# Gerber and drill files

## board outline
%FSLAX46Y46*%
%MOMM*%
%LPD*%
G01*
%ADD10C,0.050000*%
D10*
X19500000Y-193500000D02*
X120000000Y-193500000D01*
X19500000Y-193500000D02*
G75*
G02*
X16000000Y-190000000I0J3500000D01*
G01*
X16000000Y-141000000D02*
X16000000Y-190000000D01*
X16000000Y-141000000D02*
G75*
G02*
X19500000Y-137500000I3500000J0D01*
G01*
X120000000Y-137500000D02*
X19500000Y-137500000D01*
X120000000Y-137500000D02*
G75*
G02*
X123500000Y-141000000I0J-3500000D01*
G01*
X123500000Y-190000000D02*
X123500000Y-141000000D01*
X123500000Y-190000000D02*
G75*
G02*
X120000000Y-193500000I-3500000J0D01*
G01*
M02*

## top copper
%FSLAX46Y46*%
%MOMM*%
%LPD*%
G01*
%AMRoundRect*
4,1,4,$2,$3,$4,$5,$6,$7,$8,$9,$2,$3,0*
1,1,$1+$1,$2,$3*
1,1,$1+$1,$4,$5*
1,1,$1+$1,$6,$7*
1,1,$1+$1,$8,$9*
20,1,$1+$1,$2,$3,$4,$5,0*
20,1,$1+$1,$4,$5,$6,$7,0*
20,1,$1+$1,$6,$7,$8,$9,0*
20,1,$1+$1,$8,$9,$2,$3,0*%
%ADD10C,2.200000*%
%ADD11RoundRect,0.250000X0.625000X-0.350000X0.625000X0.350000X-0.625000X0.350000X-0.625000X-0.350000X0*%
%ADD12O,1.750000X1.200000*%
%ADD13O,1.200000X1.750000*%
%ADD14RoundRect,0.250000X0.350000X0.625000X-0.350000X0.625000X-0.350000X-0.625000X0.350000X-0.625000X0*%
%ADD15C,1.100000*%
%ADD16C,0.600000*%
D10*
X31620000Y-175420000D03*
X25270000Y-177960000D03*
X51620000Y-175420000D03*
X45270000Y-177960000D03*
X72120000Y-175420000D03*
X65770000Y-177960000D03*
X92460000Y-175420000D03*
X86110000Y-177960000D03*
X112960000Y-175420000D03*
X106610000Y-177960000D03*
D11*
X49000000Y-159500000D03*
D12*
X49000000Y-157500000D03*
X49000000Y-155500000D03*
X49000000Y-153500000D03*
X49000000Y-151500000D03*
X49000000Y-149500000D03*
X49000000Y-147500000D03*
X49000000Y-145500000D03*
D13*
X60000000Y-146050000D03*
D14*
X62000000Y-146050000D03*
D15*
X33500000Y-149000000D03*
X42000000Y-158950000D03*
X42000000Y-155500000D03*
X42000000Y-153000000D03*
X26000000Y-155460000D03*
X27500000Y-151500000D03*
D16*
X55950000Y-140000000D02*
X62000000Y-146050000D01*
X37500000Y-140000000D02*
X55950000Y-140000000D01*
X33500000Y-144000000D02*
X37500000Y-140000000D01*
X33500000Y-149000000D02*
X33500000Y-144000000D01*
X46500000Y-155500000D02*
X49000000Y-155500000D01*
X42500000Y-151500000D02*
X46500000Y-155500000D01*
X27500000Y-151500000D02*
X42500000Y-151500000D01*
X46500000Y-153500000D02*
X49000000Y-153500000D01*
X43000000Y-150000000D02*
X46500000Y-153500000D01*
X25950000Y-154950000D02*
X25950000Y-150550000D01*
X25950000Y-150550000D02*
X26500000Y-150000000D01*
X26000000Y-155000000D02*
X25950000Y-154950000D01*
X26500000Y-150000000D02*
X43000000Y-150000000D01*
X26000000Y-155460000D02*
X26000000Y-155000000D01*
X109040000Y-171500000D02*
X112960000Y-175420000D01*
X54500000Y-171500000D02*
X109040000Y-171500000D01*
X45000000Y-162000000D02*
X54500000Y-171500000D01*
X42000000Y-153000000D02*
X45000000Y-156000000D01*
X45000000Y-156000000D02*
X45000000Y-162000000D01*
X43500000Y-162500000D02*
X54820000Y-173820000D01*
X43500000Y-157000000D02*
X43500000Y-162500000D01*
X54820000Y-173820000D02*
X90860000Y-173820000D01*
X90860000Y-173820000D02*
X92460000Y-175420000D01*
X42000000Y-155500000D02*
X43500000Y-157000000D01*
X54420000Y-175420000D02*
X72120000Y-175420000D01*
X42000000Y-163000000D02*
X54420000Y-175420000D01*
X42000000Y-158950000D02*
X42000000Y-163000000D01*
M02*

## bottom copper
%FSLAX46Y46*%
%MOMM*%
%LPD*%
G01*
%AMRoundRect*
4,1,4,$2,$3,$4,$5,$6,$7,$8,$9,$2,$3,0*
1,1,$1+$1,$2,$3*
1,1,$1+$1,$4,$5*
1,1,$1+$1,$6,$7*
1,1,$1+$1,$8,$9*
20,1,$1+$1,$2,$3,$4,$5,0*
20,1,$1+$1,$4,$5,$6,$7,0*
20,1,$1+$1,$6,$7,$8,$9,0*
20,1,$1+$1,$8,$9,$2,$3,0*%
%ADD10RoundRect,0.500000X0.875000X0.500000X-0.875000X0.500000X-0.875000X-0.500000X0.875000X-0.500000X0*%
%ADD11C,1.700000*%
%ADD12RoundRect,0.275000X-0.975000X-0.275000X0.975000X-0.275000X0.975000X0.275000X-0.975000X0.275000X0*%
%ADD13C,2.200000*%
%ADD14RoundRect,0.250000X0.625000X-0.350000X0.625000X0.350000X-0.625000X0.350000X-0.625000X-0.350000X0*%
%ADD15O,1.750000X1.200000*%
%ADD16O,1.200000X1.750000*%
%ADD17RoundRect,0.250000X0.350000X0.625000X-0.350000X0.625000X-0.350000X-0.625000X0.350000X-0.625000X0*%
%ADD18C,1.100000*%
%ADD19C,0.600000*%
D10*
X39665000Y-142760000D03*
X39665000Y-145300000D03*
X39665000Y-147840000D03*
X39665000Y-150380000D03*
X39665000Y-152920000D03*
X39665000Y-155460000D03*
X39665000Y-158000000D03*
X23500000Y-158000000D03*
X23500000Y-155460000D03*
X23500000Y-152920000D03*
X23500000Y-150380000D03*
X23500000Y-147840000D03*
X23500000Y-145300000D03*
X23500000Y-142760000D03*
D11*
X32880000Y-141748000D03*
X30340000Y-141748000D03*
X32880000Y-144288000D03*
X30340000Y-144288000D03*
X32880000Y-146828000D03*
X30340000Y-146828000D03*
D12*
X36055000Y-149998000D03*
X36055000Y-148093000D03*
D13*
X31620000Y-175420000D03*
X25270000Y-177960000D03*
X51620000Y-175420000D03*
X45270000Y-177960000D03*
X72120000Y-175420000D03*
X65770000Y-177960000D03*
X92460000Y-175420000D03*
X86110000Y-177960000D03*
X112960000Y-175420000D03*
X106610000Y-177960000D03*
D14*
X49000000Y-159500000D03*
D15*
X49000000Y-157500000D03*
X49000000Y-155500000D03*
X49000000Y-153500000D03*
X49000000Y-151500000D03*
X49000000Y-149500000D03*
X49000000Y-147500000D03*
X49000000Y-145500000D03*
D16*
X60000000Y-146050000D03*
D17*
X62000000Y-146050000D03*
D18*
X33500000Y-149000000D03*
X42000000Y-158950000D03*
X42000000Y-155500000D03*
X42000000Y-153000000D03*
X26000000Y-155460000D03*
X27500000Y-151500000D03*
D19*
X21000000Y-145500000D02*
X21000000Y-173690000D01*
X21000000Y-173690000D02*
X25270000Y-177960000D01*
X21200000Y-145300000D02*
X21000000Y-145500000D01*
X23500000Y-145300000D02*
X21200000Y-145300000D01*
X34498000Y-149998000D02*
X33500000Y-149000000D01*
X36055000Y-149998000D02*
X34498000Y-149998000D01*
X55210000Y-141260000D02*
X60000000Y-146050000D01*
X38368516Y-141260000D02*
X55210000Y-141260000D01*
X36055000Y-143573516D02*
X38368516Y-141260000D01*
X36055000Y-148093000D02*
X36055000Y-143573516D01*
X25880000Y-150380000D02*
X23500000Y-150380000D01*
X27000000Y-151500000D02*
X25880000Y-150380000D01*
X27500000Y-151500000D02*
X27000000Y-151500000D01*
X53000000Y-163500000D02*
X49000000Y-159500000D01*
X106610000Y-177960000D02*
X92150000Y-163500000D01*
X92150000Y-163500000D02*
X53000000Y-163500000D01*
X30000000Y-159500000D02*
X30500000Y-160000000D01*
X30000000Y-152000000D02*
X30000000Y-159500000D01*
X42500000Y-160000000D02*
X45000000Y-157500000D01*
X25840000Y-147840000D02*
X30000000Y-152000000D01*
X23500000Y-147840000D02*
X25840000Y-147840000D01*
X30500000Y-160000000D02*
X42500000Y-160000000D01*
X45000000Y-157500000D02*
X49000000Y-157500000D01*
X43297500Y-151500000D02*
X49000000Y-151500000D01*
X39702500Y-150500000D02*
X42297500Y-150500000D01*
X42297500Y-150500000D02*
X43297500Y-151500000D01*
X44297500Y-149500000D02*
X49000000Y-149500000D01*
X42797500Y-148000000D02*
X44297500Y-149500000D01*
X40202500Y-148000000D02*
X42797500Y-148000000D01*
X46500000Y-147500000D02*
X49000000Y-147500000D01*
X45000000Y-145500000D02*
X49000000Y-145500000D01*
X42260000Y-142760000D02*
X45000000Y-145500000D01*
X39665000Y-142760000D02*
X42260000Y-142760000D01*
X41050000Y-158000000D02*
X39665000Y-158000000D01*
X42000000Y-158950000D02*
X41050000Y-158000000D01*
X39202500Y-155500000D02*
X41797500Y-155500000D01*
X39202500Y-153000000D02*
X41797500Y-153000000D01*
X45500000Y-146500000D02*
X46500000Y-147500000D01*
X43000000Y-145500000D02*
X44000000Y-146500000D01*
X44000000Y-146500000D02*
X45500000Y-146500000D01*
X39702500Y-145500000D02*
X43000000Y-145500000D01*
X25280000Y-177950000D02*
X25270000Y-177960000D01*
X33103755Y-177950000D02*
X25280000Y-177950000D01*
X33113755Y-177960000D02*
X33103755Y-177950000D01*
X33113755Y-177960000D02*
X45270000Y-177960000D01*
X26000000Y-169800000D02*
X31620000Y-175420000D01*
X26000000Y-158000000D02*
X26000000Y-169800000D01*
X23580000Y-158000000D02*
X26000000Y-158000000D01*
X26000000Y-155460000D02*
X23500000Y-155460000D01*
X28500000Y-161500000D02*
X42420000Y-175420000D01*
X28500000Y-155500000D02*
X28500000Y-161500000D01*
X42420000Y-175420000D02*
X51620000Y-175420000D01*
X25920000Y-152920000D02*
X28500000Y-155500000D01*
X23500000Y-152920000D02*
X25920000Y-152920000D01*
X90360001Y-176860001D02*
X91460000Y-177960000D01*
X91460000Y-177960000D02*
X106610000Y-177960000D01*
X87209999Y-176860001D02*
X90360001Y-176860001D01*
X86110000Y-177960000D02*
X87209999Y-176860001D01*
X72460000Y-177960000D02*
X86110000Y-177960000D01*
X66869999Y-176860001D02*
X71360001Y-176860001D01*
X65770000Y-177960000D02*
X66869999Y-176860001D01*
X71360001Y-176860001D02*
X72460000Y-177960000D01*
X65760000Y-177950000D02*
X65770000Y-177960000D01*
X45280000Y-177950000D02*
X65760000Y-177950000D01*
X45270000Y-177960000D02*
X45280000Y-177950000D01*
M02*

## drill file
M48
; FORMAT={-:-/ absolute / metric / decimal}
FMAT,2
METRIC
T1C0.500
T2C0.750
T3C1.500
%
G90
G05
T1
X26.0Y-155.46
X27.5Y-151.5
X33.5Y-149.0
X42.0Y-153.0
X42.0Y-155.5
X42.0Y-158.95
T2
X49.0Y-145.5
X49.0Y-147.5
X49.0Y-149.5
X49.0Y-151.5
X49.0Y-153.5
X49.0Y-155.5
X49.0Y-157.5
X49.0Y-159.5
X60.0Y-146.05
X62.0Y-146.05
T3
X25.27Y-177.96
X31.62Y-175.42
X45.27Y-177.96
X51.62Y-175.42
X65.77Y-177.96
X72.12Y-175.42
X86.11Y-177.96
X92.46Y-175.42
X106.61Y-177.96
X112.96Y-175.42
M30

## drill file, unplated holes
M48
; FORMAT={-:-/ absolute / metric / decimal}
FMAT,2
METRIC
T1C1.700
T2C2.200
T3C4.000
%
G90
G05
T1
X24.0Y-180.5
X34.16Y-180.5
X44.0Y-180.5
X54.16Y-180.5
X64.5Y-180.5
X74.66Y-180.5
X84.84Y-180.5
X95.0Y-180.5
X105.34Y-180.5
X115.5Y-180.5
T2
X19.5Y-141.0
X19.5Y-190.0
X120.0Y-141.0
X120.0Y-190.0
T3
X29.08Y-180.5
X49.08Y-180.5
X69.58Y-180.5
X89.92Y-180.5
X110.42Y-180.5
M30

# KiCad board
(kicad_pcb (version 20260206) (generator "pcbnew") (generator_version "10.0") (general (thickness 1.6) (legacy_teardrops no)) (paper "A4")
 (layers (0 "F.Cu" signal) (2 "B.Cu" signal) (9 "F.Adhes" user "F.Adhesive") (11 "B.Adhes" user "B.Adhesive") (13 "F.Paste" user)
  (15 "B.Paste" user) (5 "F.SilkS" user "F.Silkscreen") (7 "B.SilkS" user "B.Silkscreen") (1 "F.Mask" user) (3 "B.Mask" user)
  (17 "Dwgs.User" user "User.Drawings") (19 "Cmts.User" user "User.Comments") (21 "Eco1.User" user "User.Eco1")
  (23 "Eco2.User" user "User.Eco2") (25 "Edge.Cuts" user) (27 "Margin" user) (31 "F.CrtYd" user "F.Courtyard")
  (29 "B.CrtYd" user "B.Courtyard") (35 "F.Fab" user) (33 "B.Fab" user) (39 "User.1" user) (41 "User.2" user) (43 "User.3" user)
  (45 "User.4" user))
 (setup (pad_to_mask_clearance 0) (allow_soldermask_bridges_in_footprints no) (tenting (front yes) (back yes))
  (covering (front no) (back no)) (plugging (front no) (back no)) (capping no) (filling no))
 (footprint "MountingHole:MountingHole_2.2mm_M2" (layer "F.Cu") (at 120 190)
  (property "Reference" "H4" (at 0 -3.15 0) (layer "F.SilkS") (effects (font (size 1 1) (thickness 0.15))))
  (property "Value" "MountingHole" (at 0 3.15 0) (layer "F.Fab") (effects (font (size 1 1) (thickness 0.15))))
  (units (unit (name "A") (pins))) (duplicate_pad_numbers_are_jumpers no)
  (pad "" np_thru_hole circle (at 0 0) (size 2.2 2.2) (drill 2.2) (layers "*.Cu" "*.Mask")))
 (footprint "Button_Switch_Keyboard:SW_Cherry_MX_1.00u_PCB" (layer "F.Cu") (at 72.12 175.42)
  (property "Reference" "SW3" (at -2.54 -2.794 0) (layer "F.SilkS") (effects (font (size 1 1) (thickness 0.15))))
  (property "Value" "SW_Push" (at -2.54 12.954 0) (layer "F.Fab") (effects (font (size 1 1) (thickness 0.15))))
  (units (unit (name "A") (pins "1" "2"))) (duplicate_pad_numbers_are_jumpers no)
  (pad "" np_thru_hole circle (at -7.62 5.08) (size 1.7 1.7) (drill 1.7) (layers "*.Cu" "*.Mask"))
  (pad "" np_thru_hole circle (at -2.54 5.08) (size 4 4) (drill 4) (layers "*.Cu" "*.Mask"))
  (pad "" np_thru_hole circle (at 2.54 5.08) (size 1.7 1.7) (drill 1.7) (layers "*.Cu" "*.Mask"))
  (pad "1" thru_hole circle (at 0 0) (size 2.2 2.2) (drill 1.5) (layers "*.Cu" "*.Mask") (remove_unused_layers no) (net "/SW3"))
  (pad "2" thru_hole circle (at -6.35 2.54) (size 2.2 2.2) (drill 1.5) (layers "*.Cu" "*.Mask") (remove_unused_layers no) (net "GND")))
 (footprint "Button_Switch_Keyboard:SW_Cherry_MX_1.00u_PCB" (layer "F.Cu") (at 112.96 175.42)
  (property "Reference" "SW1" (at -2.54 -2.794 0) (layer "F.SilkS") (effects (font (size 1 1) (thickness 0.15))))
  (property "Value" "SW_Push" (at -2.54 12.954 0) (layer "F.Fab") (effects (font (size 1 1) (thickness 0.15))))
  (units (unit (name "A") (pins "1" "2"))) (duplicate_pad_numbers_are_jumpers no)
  (pad "" np_thru_hole circle (at -7.62 5.08) (size 1.7 1.7) (drill 1.7) (layers "*.Cu" "*.Mask"))
  (pad "" np_thru_hole circle (at -2.54 5.08) (size 4 4) (drill 4) (layers "*.Cu" "*.Mask"))
  (pad "" np_thru_hole circle (at 2.54 5.08) (size 1.7 1.7) (drill 1.7) (layers "*.Cu" "*.Mask"))
  (pad "1" thru_hole circle (at 0 0) (size 2.2 2.2) (drill 1.5) (layers "*.Cu" "*.Mask") (remove_unused_layers no) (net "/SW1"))
  (pad "2" thru_hole circle (at -6.35 2.54) (size 2.2 2.2) (drill 1.5) (layers "*.Cu" "*.Mask") (remove_unused_layers no) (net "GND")))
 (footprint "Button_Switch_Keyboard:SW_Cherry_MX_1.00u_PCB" (layer "F.Cu") (at 51.62 175.42)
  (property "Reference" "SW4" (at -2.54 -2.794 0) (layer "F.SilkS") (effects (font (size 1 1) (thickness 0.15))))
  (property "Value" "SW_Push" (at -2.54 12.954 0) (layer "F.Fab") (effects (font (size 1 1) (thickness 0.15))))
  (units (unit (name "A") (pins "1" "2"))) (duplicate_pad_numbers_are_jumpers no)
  (pad "" np_thru_hole circle (at -7.62 5.08) (size 1.7 1.7) (drill 1.7) (layers "*.Cu" "*.Mask"))
  (pad "" np_thru_hole circle (at -2.54 5.08) (size 4 4) (drill 4) (layers "*.Cu" "*.Mask"))
  (pad "" np_thru_hole circle (at 2.54 5.08) (size 1.7 1.7) (drill 1.7) (layers "*.Cu" "*.Mask"))
  (pad "1" thru_hole circle (at 0 0) (size 2.2 2.2) (drill 1.5) (layers "*.Cu" "*.Mask") (remove_unused_layers no) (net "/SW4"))
  (pad "2" thru_hole circle (at -6.35 2.54) (size 2.2 2.2) (drill 1.5) (layers "*.Cu" "*.Mask") (remove_unused_layers no) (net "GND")))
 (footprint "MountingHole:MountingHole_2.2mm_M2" (layer "F.Cu") (at 19.5 190)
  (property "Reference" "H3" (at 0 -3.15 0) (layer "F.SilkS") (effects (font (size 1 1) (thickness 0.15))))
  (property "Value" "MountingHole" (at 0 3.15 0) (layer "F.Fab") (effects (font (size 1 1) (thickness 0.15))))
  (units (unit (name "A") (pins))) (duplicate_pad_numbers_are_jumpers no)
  (pad "" np_thru_hole circle (at 0 0) (size 2.2 2.2) (drill 2.2) (layers "*.Cu" "*.Mask")))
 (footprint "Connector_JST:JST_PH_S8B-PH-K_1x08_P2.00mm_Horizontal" (layer "F.Cu") (at 49 159.5 90)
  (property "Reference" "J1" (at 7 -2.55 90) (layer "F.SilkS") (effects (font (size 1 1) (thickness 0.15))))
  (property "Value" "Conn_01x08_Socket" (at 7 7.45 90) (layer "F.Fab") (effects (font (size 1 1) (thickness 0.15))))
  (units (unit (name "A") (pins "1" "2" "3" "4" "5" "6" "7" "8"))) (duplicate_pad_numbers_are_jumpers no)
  (pad "1" thru_hole roundrect (at 0 0 90) (size 1.2 1.75) (drill 0.75) (layers "*.Cu" "*.Mask") (remove_unused_layers no)
   (roundrect_rratio 0.208333) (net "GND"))
  (pad "2" thru_hole oval (at 2 0 90) (size 1.2 1.75) (drill 0.75) (layers "*.Cu" "*.Mask") (remove_unused_layers no) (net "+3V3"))
  (pad "3" thru_hole oval (at 4 0 90) (size 1.2 1.75) (drill 0.75) (layers "*.Cu" "*.Mask") (remove_unused_layers no) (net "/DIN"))
  (pad "4" thru_hole oval (at 6 0 90) (size 1.2 1.75) (drill 0.75) (layers "*.Cu" "*.Mask") (remove_unused_layers no) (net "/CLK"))
  (pad "5" thru_hole oval (at 8 0 90) (size 1.2 1.75) (drill 0.75) (layers "*.Cu" "*.Mask") (remove_unused_layers no) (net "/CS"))
  (pad "6" thru_hole oval (at 10 0 90) (size 1.2 1.75) (drill 0.75) (layers "*.Cu" "*.Mask") (remove_unused_layers no) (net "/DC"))
  (pad "7" thru_hole oval (at 12 0 90) (size 1.2 1.75) (drill 0.75) (layers "*.Cu" "*.Mask") (remove_unused_layers no) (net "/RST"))
  (pad "8" thru_hole oval (at 14 0 90) (size 1.2 1.75) (drill 0.75) (layers "*.Cu" "*.Mask") (remove_unused_layers no) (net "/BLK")))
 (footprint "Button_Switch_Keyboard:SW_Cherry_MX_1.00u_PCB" (layer "F.Cu") (at 31.62 175.42)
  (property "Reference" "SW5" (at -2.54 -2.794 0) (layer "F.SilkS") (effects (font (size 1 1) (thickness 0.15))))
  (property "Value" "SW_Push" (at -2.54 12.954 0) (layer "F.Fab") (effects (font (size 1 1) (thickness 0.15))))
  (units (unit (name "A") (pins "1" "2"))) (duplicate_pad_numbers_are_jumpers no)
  (pad "" np_thru_hole circle (at -7.62 5.08) (size 1.7 1.7) (drill 1.7) (layers "*.Cu" "*.Mask"))
  (pad "" np_thru_hole circle (at -2.54 5.08) (size 4 4) (drill 4) (layers "*.Cu" "*.Mask"))
  (pad "" np_thru_hole circle (at 2.54 5.08) (size 1.7 1.7) (drill 1.7) (layers "*.Cu" "*.Mask"))
  (pad "1" thru_hole circle (at 0 0) (size 2.2 2.2) (drill 1.5) (layers "*.Cu" "*.Mask") (remove_unused_layers no) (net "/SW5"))
  (pad "2" thru_hole circle (at -6.35 2.54) (size 2.2 2.2) (drill 1.5) (layers "*.Cu" "*.Mask") (remove_unused_layers no) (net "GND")))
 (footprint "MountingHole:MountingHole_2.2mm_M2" (layer "F.Cu") (at 120 141)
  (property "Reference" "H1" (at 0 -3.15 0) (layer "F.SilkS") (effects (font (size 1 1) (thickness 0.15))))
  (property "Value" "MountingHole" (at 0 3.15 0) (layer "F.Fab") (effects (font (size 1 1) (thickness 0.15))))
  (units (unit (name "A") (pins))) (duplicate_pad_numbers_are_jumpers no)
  (pad "" np_thru_hole circle (at 0 0) (size 2.2 2.2) (drill 2.2) (layers "*.Cu" "*.Mask")))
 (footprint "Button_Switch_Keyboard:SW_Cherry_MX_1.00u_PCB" (layer "F.Cu") (at 92.46 175.42)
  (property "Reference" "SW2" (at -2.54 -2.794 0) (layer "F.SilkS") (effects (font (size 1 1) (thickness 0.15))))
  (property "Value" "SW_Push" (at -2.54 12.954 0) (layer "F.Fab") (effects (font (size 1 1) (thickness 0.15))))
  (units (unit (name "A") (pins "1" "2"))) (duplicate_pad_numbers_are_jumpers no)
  (pad "" np_thru_hole circle (at -7.62 5.08) (size 1.7 1.7) (drill 1.7) (layers "*.Cu" "*.Mask"))
  (pad "" np_thru_hole circle (at -2.54 5.08) (size 4 4) (drill 4) (layers "*.Cu" "*.Mask"))
  (pad "" np_thru_hole circle (at 2.54 5.08) (size 1.7 1.7) (drill 1.7) (layers "*.Cu" "*.Mask"))
  (pad "1" thru_hole circle (at 0 0) (size 2.2 2.2) (drill 1.5) (layers "*.Cu" "*.Mask") (remove_unused_layers no) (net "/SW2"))
  (pad "2" thru_hole circle (at -6.35 2.54) (size 2.2 2.2) (drill 1.5) (layers "*.Cu" "*.Mask") (remove_unused_layers no) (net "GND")))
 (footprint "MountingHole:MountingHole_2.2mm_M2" (layer "F.Cu") (at 19.5 141)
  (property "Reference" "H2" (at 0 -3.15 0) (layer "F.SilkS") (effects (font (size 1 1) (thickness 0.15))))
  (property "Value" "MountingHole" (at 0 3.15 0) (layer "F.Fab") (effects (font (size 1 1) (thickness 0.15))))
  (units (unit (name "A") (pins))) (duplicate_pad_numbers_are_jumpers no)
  (pad "" np_thru_hole circle (at 0 0) (size 2.2 2.2) (drill 2.2) (layers "*.Cu" "*.Mask")))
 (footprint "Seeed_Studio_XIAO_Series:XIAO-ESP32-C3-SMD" (layer "B.Cu") (at 40.5 160.88 180)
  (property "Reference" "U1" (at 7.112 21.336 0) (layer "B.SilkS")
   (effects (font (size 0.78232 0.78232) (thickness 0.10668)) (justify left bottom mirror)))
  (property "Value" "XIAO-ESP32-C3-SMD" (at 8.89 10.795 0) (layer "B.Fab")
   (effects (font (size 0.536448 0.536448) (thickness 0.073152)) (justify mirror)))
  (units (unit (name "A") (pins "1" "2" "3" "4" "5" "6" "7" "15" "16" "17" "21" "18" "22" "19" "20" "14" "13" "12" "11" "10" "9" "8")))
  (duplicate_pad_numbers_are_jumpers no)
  (pad "1" smd roundrect (at 0.835 18.12 180) (size 2.75 2) (layers "B.Cu" "B.Mask" "B.Paste") (roundrect_rratio 0.25) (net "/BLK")
   (solder_mask_margin 0.0508) (thermal_bridge_angle 45))
  (pad "2" smd roundrect (at 0.835 15.58 180) (size 2.75 2) (layers "B.Cu" "B.Mask" "B.Paste") (roundrect_rratio 0.25) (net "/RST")
   (solder_mask_margin 0.0508) (thermal_bridge_angle 45))
  (pad "3" smd roundrect (at 0.835 13.04 180) (size 2.75 2) (layers "B.Cu" "B.Mask" "B.Paste") (roundrect_rratio 0.25) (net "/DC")
   (solder_mask_margin 0.0508) (thermal_bridge_angle 45))
  (pad "4" smd roundrect (at 0.835 10.5 180) (size 2.75 2) (layers "B.Cu" "B.Mask" "B.Paste") (roundrect_rratio 0.25) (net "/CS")
   (solder_mask_margin 0.0508) (thermal_bridge_angle 45))
  (pad "5" smd roundrect (at 0.835 7.96 180) (size 2.75 2) (layers "B.Cu" "B.Mask" "B.Paste") (roundrect_rratio 0.25) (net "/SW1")
   (solder_mask_margin 0.0508) (thermal_bridge_angle 45))
  (pad "6" smd roundrect (at 0.835 5.42 180) (size 2.75 2) (layers "B.Cu" "B.Mask" "B.Paste") (roundrect_rratio 0.25) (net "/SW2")
   (solder_mask_margin 0.0508) (thermal_bridge_angle 45))
  (pad "7" smd roundrect (at 0.835 2.88 180) (size 2.75 2) (layers "B.Cu" "B.Mask" "B.Paste") (roundrect_rratio 0.25) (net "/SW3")
   (solder_mask_margin 0.0508) (thermal_bridge_angle 45))
  (pad "8" smd roundrect (at 17 2.88 180) (size 2.75 2) (layers "B.Cu" "B.Mask" "B.Paste") (roundrect_rratio 0.25) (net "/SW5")
   (solder_mask_margin 0.0508) (thermal_bridge_angle 45))
  (pad "9" smd roundrect (at 17 5.42 180) (size 2.75 2) (layers "B.Cu" "B.Mask" "B.Paste") (roundrect_rratio 0.25) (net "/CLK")
   (solder_mask_margin 0.0508) (thermal_bridge_angle 45))
  (pad "10" smd roundrect (at 17 7.96 180) (size 2.75 2) (layers "B.Cu" "B.Mask" "B.Paste") (roundrect_rratio 0.25) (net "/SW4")
   (solder_mask_margin 0.0508) (thermal_bridge_angle 45))
  (pad "11" smd roundrect (at 17 10.5 180) (size 2.75 2) (layers "B.Cu" "B.Mask" "B.Paste") (roundrect_rratio 0.25) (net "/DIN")
   (solder_mask_margin 0.0508) (thermal_bridge_angle 45))
  (pad "12" smd roundrect (at 17 13.04 180) (size 2.75 2) (layers "B.Cu" "B.Mask" "B.Paste") (roundrect_rratio 0.25) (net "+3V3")
   (solder_mask_margin 0.0508) (thermal_bridge_angle 45))
  (pad "13" smd roundrect (at 17 15.58 180) (size 2.75 2) (layers "B.Cu" "B.Mask" "B.Paste") (roundrect_rratio 0.25) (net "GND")
   (solder_mask_margin 0.0508) (thermal_bridge_angle 45))
  (pad "14" smd roundrect (at 17 18.12 180) (size 2.75 2) (layers "B.Cu" "B.Mask" "B.Paste") (roundrect_rratio 0.25)
   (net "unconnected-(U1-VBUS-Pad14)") (solder_mask_margin 0.0508) (thermal_bridge_angle 45))
  (pad "15" smd circle (at 7.62 19.132 180) (size 1.7 1.7) (layers "B.Cu" "B.Mask" "B.Paste") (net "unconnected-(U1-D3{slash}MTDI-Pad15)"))
  (pad "16" smd circle (at 10.16 19.132 180) (size 1.7 1.7) (layers "B.Cu" "B.Mask" "B.Paste") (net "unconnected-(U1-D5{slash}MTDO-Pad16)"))
  (pad "17" smd circle (at 7.62 16.592 180) (size 1.7 1.7) (layers "B.Cu" "B.Mask" "B.Paste") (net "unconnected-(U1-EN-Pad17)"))
  (pad "18" smd circle (at 10.16 16.592 180) (size 1.7 1.7) (layers "B.Cu" "B.Mask" "B.Paste") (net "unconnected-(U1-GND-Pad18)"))
  (pad "19" smd circle (at 7.62 14.052 180) (size 1.7 1.7) (layers "B.Cu" "B.Mask" "B.Paste") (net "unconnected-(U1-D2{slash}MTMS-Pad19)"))
  (pad "20" smd circle (at 10.16 14.052 180) (size 1.7 1.7) (layers "B.Cu" "B.Mask" "B.Paste") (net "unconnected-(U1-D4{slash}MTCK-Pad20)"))
  (pad "21" smd roundrect (at 4.445 10.882) (size 2.5 1.1) (layers "B.Cu" "B.Mask" "B.Paste") (roundrect_rratio 0.25) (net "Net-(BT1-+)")
   (thermal_bridge_angle 45))
  (pad "22" smd roundrect (at 4.445 12.787) (size 2.5 1.1) (layers "B.Cu" "B.Mask" "B.Paste") (roundrect_rratio 0.25) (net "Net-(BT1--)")
   (thermal_bridge_angle 45)))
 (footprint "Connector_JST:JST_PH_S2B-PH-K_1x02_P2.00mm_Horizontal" (layer "B.Cu") (at 62 146.05 180)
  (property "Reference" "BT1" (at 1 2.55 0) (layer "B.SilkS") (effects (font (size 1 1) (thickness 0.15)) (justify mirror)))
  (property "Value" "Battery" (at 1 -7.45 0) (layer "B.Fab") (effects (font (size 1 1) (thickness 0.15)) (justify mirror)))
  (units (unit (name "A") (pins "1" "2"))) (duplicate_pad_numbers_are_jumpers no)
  (pad "1" thru_hole roundrect (at 0 0 180) (size 1.2 1.75) (drill 0.75) (layers "*.Cu" "*.Mask") (remove_unused_layers no)
   (roundrect_rratio 0.208333) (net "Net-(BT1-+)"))
  (pad "2" thru_hole oval (at 2 0 180) (size 1.2 1.75) (drill 0.75) (layers "*.Cu" "*.Mask") (remove_unused_layers no) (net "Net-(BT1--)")))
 (gr_line (start 16 141) (end 16 190) (stroke (width 0.05) (type default)) (layer "Edge.Cuts"))
 (gr_arc (start 16 141) (mid 17.025126 138.525126) (end 19.5 137.5) (stroke (width 0.05) (type default)) (layer "Edge.Cuts"))
 (gr_arc (start 19.5 193.5) (mid 17.025126 192.474874) (end 16 190) (stroke (width 0.05) (type default)) (layer "Edge.Cuts"))
 (gr_line (start 19.5 193.5) (end 120 193.5) (stroke (width 0.05) (type default)) (layer "Edge.Cuts"))
 (gr_line (start 120 137.5) (end 19.5 137.5) (stroke (width 0.05) (type default)) (layer "Edge.Cuts"))
 (gr_arc (start 120 137.5) (mid 122.474874 138.525126) (end 123.5 141) (stroke (width 0.05) (type default)) (layer "Edge.Cuts"))
 (gr_arc (start 123.5 190) (mid 122.474874 192.474874) (end 120 193.5) (stroke (width 0.05) (type default)) (layer "Edge.Cuts"))
 (gr_line (start 123.5 190) (end 123.5 141) (stroke (width 0.05) (type default)) (layer "Edge.Cuts"))
 (segment (start 42 158.95) (end 42 163) (width 0.6) (layer "F.Cu") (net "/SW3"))
 (segment (start 54.42 175.42) (end 72.12 175.42) (width 0.6) (layer "F.Cu") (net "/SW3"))
 (segment (start 42 163) (end 54.42 175.42) (width 0.6) (layer "F.Cu") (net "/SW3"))
 (via (at 42 158.95) (size 1.1) (drill 0.5) (layers "F.Cu" "B.Cu") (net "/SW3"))
 (segment (start 41.05 158) (end 39.665 158) (width 0.6) (layer "B.Cu") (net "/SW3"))
 (segment (start 42 158.95) (end 41.05 158) (width 0.6) (layer "B.Cu") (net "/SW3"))
 (segment (start 72.46 177.96) (end 86.11 177.96) (width 0.6) (layer "B.Cu") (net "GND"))
 (segment (start 33.113755 177.96) (end 33.103755 177.95) (width 0.6) (layer "B.Cu") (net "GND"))
 (segment (start 71.360001 176.860001) (end 72.46 177.96) (width 0.6) (layer "B.Cu") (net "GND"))
 (segment (start 92.15 163.5) (end 53 163.5) (width 0.6) (layer "B.Cu") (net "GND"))
 (segment (start 53 163.5) (end 49 159.5) (width 0.6) (layer "B.Cu") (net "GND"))
 (segment (start 66.869999 176.860001) (end 71.360001 176.860001) (width 0.6) (layer "B.Cu") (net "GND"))
 (segment (start 65.76 177.95) (end 65.77 177.96) (width 0.6) (layer "B.Cu") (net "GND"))
 (segment (start 45.28 177.95) (end 65.76 177.95) (width 0.6) (layer "B.Cu") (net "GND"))
 (segment (start 33.103755 177.95) (end 25.28 177.95) (width 0.6) (layer "B.Cu") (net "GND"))
 (segment (start 87.209999 176.860001) (end 90.360001 176.860001) (width 0.6) (layer "B.Cu") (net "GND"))
 (segment (start 90.360001 176.860001) (end 91.46 177.96) (width 0.6) (layer "B.Cu") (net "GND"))
 (segment (start 21 173.69) (end 25.27 177.96) (width 0.6) (layer "B.Cu") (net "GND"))
 (segment (start 21.2 145.3) (end 21 145.5) (width 0.6) (layer "B.Cu") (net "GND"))
 (segment (start 33.113755 177.96) (end 45.27 177.96) (width 0.6) (layer "B.Cu") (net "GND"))
 (segment (start 91.46 177.96) (end 106.61 177.96) (width 0.6) (layer "B.Cu") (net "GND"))
 (segment (start 45.27 177.96) (end 45.28 177.95) (width 0.6) (layer "B.Cu") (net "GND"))
 (segment (start 25.28 177.95) (end 25.27 177.96) (width 0.6) (layer "B.Cu") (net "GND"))
 (segment (start 106.61 177.96) (end 92.15 163.5) (width 0.6) (layer "B.Cu") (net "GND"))
 (segment (start 86.11 177.96) (end 87.209999 176.860001) (width 0.6) (layer "B.Cu") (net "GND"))
 (segment (start 21 145.5) (end 21 173.69) (width 0.6) (layer "B.Cu") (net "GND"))
 (segment (start 65.77 177.96) (end 66.869999 176.860001) (width 0.6) (layer "B.Cu") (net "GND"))
 (segment (start 23.5 145.3) (end 21.2 145.3) (width 0.6) (layer "B.Cu") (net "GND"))
 (segment (start 26 169.8) (end 31.62 175.42) (width 0.6) (layer "B.Cu") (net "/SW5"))
 (segment (start 23.58 158) (end 26 158) (width 0.6) (layer "B.Cu") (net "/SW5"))
 (segment (start 26 158) (end 26 169.8) (width 0.6) (layer "B.Cu") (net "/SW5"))
 (segment (start 43.5 157) (end 43.5 162.5) (width 0.6) (layer "F.Cu") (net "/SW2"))
 (segment (start 42 155.5) (end 43.5 157) (width 0.6) (layer "F.Cu") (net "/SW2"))
 (segment (start 43.5 162.5) (end 54.82 173.82) (width 0.6) (layer "F.Cu") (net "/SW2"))
 (segment (start 54.82 173.82) (end 90.86 173.82) (width 0.6) (layer "F.Cu") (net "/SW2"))
 (segment (start 90.86 173.82) (end 92.46 175.42) (width 0.6) (layer "F.Cu") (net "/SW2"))
 (via (at 42 155.5) (size 1.1) (drill 0.5) (layers "F.Cu" "B.Cu") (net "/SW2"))
 (segment (start 39.2025 155.5) (end 41.7975 155.5) (width 0.6) (layer "B.Cu") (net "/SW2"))
 (segment (start 45 156) (end 45 162) (width 0.6) (layer "F.Cu") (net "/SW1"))
 (segment (start 54.5 171.5) (end 109.04 171.5) (width 0.6) (layer "F.Cu") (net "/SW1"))
 (segment (start 45 162) (end 54.5 171.5) (width 0.6) (layer "F.Cu") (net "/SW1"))
 (segment (start 109.04 171.5) (end 112.96 175.42) (width 0.6) (layer "F.Cu") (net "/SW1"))
 (segment (start 42 153) (end 45 156) (width 0.6) (layer "F.Cu") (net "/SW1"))
 (via (at 42 153) (size 1.1) (drill 0.5) (layers "F.Cu" "B.Cu") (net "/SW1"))
 (segment (start 39.2025 153) (end 41.7975 153) (width 0.6) (layer "B.Cu") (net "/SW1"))
 (segment (start 28.5 155.5) (end 28.5 161.5) (width 0.6) (layer "B.Cu") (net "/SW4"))
 (segment (start 23.5 152.92) (end 25.92 152.92) (width 0.6) (layer "B.Cu") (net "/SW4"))
 (segment (start 25.92 152.92) (end 28.5 155.5) (width 0.6) (layer "B.Cu") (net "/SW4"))
 (segment (start 28.5 161.5) (end 42.42 175.42) (width 0.6) (layer "B.Cu") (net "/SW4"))
 (segment (start 42.42 175.42) (end 51.62 175.42) (width 0.6) (layer "B.Cu") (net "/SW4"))
 (segment (start 30.5 160) (end 42.5 160) (width 0.6) (layer "B.Cu") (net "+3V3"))
 (segment (start 30 152) (end 30 159.5) (width 0.6) (layer "B.Cu") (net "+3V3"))
 (segment (start 30 159.5) (end 30.5 160) (width 0.6) (layer "B.Cu") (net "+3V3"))
 (segment (start 25.84 147.84) (end 30 152) (width 0.6) (layer "B.Cu") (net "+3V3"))
 (segment (start 45 157.5) (end 49 157.5) (width 0.6) (layer "B.Cu") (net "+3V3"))
 (segment (start 23.5 147.84) (end 25.84 147.84) (width 0.6) (layer "B.Cu") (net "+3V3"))
 (segment (start 42.5 160) (end 45 157.5) (width 0.6) (layer "B.Cu") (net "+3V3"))
 (segment (start 27.5 151.5) (end 42.5 151.5) (width 0.6) (layer "F.Cu") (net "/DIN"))
 (segment (start 46.5 155.5) (end 49 155.5) (width 0.6) (layer "F.Cu") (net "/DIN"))
 (segment (start 42.5 151.5) (end 46.5 155.5) (width 0.6) (layer "F.Cu") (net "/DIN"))
 (via (at 27.5 151.5) (size 1.1) (drill 0.5) (layers "F.Cu" "B.Cu") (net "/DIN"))
 (segment (start 27.5 151.5) (end 27 151.5) (width 0.6) (layer "B.Cu") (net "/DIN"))
 (segment (start 27 151.5) (end 25.88 150.38) (width 0.6) (layer "B.Cu") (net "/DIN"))
 (segment (start 25.88 150.38) (end 23.5 150.38) (width 0.6) (layer "B.Cu") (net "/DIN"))
 (segment (start 46.5 153.5) (end 49 153.5) (width 0.6) (layer "F.Cu") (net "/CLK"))
 (segment (start 26 155.46) (end 26 155) (width 0.6) (layer "F.Cu") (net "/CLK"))
 (segment (start 25.95 150.55) (end 26.5 150) (width 0.6) (layer "F.Cu") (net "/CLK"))
 (segment (start 43 150) (end 46.5 153.5) (width 0.6) (layer "F.Cu") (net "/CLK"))
 (segment (start 26.5 150) (end 43 150) (width 0.6) (layer "F.Cu") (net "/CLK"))
 (segment (start 26 155) (end 25.95 154.95) (width 0.6) (layer "F.Cu") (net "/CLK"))
 (segment (start 25.95 154.95) (end 25.95 150.55) (width 0.6) (layer "F.Cu") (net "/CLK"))
 (via (at 26 155.46) (size 1.1) (drill 0.5) (layers "F.Cu" "B.Cu") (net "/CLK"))
 (segment (start 26 155.46) (end 23.5 155.46) (width 0.6) (layer "B.Cu") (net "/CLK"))
 (segment (start 43.2975 151.5) (end 49 151.5) (width 0.6) (layer "B.Cu") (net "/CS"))
 (segment (start 42.2975 150.5) (end 43.2975 151.5) (width 0.6) (layer "B.Cu") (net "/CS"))
 (segment (start 39.7025 150.5) (end 42.2975 150.5) (width 0.6) (layer "B.Cu") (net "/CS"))
 (segment (start 44.2975 149.5) (end 49 149.5) (width 0.6) (layer "B.Cu") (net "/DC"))
 (segment (start 42.7975 148) (end 44.2975 149.5) (width 0.6) (layer "B.Cu") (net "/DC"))
 (segment (start 40.2025 148) (end 42.7975 148) (width 0.6) (layer "B.Cu") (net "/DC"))
 (segment (start 44 146.5) (end 45.5 146.5) (width 0.6) (layer "B.Cu") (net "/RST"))
 (segment (start 39.7025 145.5) (end 43 145.5) (width 0.6) (layer "B.Cu") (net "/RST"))
 (segment (start 45.5 146.5) (end 46.5 147.5) (width 0.6) (layer "B.Cu") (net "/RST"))
 (segment (start 43 145.5) (end 44 146.5) (width 0.6) (layer "B.Cu") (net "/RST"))
 (segment (start 46.5 147.5) (end 49 147.5) (width 0.6) (layer "B.Cu") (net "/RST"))
 (segment (start 39.665 142.76) (end 42.26 142.76) (width 0.6) (layer "B.Cu") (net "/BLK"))
 (segment (start 45 145.5) (end 49 145.5) (width 0.6) (layer "B.Cu") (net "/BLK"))
 (segment (start 42.26 142.76) (end 45 145.5) (width 0.6) (layer "B.Cu") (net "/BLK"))
 (segment (start 37.5 140) (end 55.95 140) (width 0.6) (layer "F.Cu") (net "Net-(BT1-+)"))
 (segment (start 33.5 149) (end 33.5 144) (width 0.6) (layer "F.Cu") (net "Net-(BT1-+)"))
 (segment (start 55.95 140) (end 62 146.05) (width 0.6) (layer "F.Cu") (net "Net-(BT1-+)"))
 (segment (start 33.5 144) (end 37.5 140) (width 0.6) (layer "F.Cu") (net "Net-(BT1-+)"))
 (via (at 33.5 149) (size 1.1) (drill 0.5) (layers "F.Cu" "B.Cu") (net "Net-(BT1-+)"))
 (segment (start 34.498 149.998) (end 33.5 149) (width 0.6) (layer "B.Cu") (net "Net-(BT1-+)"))
 (segment (start 36.055 149.998) (end 34.498 149.998) (width 0.6) (layer "B.Cu") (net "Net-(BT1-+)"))
 (segment (start 38.368516 141.26) (end 55.21 141.26) (width 0.6) (layer "B.Cu") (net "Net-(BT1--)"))
 (segment (start 36.055 143.573516) (end 38.368516 141.26) (width 0.6) (layer "B.Cu") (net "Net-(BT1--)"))
 (segment (start 36.055 148.093) (end 36.055 143.573516) (width 0.6) (layer "B.Cu") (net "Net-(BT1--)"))
 (segment (start 55.21 141.26) (end 60 146.05) (width 0.6) (layer "B.Cu") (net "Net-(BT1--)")))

